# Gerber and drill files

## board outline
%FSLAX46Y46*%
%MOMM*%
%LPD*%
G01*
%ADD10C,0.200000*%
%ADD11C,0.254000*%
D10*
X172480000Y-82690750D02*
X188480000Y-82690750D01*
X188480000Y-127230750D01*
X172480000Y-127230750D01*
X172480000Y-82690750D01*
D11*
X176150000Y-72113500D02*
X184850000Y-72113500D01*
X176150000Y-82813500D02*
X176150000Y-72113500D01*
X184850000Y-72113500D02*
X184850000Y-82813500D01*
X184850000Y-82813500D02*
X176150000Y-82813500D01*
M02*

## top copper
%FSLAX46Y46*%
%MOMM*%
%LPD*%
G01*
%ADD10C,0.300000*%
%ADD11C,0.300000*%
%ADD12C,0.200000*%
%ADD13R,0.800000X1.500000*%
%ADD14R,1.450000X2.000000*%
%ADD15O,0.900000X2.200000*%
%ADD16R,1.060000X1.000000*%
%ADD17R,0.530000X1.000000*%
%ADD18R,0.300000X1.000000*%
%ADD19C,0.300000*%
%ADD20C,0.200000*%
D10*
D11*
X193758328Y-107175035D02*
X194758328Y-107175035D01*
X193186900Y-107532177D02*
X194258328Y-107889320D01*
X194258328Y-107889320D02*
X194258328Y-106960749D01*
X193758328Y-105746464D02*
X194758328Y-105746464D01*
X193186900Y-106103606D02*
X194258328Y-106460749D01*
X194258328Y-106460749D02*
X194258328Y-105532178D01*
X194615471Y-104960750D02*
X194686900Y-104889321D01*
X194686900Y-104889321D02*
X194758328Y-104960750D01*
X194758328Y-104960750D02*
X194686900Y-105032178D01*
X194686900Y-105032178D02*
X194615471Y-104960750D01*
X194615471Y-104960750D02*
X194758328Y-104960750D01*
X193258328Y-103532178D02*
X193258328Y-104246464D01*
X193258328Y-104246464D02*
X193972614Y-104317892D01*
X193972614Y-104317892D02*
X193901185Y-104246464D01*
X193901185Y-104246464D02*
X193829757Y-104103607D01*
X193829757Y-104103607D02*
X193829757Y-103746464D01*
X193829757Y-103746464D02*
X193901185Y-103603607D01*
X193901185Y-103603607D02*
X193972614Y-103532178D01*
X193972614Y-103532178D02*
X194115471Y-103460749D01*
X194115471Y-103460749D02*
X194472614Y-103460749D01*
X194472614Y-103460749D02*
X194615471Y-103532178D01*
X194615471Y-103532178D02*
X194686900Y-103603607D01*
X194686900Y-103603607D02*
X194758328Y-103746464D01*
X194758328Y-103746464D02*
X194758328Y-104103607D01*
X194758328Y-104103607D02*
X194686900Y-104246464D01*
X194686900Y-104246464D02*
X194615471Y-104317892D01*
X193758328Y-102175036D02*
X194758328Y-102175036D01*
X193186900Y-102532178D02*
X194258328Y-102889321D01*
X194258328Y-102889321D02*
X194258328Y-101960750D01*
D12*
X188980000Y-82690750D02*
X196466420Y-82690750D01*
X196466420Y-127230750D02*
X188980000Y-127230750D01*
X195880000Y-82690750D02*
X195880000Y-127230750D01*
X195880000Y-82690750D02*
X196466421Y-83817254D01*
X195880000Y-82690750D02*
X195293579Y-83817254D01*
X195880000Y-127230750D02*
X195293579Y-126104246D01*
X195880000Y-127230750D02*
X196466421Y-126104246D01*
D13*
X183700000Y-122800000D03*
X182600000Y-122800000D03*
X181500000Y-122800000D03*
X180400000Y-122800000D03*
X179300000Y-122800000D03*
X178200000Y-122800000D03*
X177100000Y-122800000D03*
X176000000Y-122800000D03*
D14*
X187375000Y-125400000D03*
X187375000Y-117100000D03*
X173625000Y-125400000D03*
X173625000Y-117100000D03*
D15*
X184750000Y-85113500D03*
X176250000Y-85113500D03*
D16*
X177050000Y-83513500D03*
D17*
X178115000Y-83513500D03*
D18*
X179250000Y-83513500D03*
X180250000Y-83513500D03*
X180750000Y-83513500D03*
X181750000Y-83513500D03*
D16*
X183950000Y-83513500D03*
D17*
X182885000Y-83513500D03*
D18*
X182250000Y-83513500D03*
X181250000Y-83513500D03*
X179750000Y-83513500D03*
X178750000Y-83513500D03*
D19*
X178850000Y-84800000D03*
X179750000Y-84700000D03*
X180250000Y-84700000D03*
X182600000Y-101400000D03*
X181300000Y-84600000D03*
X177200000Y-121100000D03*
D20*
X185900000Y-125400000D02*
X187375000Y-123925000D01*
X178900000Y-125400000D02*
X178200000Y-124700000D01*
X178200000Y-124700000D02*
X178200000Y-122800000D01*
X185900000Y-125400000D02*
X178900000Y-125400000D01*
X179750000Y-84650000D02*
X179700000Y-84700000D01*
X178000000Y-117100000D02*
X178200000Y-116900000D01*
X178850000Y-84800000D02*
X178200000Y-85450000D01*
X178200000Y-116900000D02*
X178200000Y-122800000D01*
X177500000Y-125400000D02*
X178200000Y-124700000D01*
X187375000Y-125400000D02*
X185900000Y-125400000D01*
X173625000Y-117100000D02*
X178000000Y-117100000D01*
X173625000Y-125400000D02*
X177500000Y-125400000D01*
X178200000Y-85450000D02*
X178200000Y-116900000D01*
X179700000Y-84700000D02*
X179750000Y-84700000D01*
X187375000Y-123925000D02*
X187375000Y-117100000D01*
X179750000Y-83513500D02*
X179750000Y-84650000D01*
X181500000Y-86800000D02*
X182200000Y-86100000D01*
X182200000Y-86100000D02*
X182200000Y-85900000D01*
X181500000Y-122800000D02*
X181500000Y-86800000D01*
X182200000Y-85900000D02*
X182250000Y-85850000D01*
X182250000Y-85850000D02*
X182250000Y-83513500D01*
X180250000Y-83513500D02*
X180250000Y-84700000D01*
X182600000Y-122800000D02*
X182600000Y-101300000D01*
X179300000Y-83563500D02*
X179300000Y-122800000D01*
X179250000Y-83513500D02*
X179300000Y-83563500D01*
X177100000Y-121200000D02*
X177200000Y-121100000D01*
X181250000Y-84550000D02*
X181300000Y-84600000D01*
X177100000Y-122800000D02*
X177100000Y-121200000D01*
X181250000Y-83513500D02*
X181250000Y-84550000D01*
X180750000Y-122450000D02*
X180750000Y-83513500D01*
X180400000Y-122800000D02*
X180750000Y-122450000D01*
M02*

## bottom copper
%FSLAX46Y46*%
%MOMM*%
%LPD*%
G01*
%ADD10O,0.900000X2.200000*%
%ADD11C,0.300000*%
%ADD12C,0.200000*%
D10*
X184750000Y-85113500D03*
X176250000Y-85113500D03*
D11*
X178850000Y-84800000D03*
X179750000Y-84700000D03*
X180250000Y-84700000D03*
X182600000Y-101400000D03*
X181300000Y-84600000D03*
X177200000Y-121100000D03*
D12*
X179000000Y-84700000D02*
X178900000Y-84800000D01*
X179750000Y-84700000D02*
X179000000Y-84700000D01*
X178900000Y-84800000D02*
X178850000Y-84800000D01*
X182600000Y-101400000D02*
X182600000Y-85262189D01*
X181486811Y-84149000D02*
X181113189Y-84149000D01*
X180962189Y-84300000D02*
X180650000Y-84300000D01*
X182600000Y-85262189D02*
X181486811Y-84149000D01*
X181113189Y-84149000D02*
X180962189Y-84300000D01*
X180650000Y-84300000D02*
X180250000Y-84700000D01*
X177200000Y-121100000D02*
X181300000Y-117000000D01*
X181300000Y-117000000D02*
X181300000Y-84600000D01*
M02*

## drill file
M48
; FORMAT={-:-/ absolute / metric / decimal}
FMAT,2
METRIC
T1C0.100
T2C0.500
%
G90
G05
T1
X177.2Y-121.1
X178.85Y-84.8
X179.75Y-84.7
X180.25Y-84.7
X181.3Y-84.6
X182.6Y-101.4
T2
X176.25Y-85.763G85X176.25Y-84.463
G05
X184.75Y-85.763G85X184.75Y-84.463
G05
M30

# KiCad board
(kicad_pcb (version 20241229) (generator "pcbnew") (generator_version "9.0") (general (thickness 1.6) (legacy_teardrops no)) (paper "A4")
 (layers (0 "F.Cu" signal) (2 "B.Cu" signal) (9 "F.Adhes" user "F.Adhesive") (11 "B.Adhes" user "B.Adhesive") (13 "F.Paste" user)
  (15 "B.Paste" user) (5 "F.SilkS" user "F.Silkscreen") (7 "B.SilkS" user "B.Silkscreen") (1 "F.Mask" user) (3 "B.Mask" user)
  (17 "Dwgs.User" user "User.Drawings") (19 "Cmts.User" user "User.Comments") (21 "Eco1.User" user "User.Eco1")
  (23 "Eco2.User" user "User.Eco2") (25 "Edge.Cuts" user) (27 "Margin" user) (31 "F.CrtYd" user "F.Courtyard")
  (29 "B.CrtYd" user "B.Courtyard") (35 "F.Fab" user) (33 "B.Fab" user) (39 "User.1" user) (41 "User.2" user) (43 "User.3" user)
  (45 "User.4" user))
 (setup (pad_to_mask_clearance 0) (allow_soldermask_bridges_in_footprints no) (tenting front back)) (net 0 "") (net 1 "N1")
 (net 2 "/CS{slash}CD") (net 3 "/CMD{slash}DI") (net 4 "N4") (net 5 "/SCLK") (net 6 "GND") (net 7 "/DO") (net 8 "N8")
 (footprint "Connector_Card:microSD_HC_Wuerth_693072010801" (layer "F.Cu") (at 180.5 121.25 180)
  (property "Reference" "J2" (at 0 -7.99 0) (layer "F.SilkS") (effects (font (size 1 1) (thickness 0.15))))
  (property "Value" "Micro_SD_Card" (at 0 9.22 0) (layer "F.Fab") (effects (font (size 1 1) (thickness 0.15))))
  (pad "1" smd rect (at -3.2 -1.55 180) (size 0.8 1.5) (layers "F.Cu" "F.Mask" "F.Paste") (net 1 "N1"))
  (pad "2" smd rect (at -2.1 -1.55 180) (size 0.8 1.5) (layers "F.Cu" "F.Mask" "F.Paste") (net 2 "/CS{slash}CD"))
  (pad "3" smd rect (at -1 -1.55 180) (size 0.8 1.5) (layers "F.Cu" "F.Mask" "F.Paste") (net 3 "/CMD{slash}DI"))
  (pad "4" smd rect (at 0.1 -1.55 180) (size 0.8 1.5) (layers "F.Cu" "F.Mask" "F.Paste") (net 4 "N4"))
  (pad "5" smd rect (at 1.2 -1.55 180) (size 0.8 1.5) (layers "F.Cu" "F.Mask" "F.Paste") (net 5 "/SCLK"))
  (pad "6" smd rect (at 2.3 -1.55 180) (size 0.8 1.5) (layers "F.Cu" "F.Mask" "F.Paste") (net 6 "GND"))
  (pad "7" smd rect (at 3.4 -1.55 180) (size 0.8 1.5) (layers "F.Cu" "F.Mask" "F.Paste") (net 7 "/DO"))
  (pad "8" smd rect (at 4.5 -1.55 180) (size 0.8 1.5) (layers "F.Cu" "F.Mask" "F.Paste") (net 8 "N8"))
  (pad "9" smd rect (at -6.875 -4.15 180) (size 1.45 2) (layers "F.Cu" "F.Mask" "F.Paste") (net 6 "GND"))
  (pad "9" smd rect (at -6.875 4.15 180) (size 1.45 2) (layers "F.Cu" "F.Mask" "F.Paste") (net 6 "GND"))
  (pad "9" smd rect (at 6.875 -4.15 180) (size 1.45 2) (layers "F.Cu" "F.Mask" "F.Paste") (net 6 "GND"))
  (pad "9" smd rect (at 6.875 4.15 180) (size 1.45 2) (layers "F.Cu" "F.Mask" "F.Paste") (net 6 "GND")))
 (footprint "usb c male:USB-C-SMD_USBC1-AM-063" (layer "F.Cu") (at 180.5 84.3135 180)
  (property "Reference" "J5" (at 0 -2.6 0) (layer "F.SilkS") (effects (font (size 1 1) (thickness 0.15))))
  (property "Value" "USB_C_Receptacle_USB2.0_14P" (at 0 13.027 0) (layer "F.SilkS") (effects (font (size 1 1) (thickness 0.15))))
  (fp_line (start 4.35 12.2) (end -4.35 12.2) (stroke (width 0.254) (type default)) (layer "Edge.Cuts"))
  (fp_line (start 4.35 1.5) (end 4.35 12.2) (stroke (width 0.254) (type default)) (layer "Edge.Cuts"))
  (fp_line (start -4.35 12.2) (end -4.35 1.5) (stroke (width 0.254) (type default)) (layer "Edge.Cuts"))
  (fp_line (start -4.35 1.5) (end 4.35 1.5) (stroke (width 0.254) (type default)) (layer "Edge.Cuts"))
  (pad "1" thru_hole oval (at -4.25 -0.8 180) (size 0.9 2.2) (drill oval 0.5 1.8) (layers "*.Cu" "*.Mask") (remove_unused_layers no))
  (pad "2" thru_hole oval (at 4.25 -0.8 180) (size 0.9 2.2) (drill oval 0.5 1.8) (layers "*.Cu" "*.Mask") (remove_unused_layers no))
  (pad "A1B12" smd rect (at 3.45 0.8) (size 1.06 1) (layers "F.Cu" "F.Mask" "F.Paste"))
  (pad "A4B9" smd rect (at 2.385 0.8) (size 0.53 1) (layers "F.Cu" "F.Mask" "F.Paste"))
  (pad "A5" smd rect (at 1.25 0.8) (size 0.3 1) (layers "F.Cu" "F.Mask" "F.Paste") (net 5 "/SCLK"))
  (pad "A6" smd rect (at 0.25 0.8 180) (size 0.3 1) (layers "F.Cu" "F.Mask" "F.Paste") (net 2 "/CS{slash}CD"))
  (pad "A7" smd rect (at -0.25 0.8) (size 0.3 1) (layers "F.Cu" "F.Mask" "F.Paste") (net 4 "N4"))
  (pad "A8" smd rect (at -1.25 0.8) (size 0.3 1) (layers "F.Cu" "F.Mask" "F.Paste"))
  (pad "B1A12" smd rect (at -3.45 0.8) (size 1.06 1) (layers "F.Cu" "F.Mask" "F.Paste"))
  (pad "B4A9" smd rect (at -2.385 0.8) (size 0.53 1) (layers "F.Cu" "F.Mask" "F.Paste"))
  (pad "B5" smd rect (at -1.75 0.8) (size 0.3 1) (layers "F.Cu" "F.Mask" "F.Paste") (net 3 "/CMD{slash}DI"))
  (pad "B6" smd rect (at -0.75 0.8 180) (size 0.3 1) (layers "F.Cu" "F.Mask" "F.Paste") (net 7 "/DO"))
  (pad "B7" smd rect (at 0.75 0.8) (size 0.3 1) (layers "F.Cu" "F.Mask" "F.Paste") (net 6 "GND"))
  (pad "B8" smd rect (at 1.75 0.8) (size 0.3 1) (layers "F.Cu" "F.Mask" "F.Paste")))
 (gr_rect (start 172.48 82.69075) (end 188.48 127.23075) (stroke (width 0.2) (type solid)) (fill no) (layer "Edge.Cuts"))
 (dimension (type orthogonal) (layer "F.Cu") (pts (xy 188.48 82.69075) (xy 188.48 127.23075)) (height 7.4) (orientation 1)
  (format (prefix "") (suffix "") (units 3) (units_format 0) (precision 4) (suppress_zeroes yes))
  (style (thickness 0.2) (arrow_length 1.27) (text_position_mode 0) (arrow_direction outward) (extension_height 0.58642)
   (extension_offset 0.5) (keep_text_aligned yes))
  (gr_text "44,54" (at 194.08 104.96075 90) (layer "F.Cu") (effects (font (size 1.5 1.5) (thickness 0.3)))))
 (segment (start 185.9 125.4) (end 187.375 123.925) (width 0.2) (layer "F.Cu") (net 6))
 (segment (start 178.9 125.4) (end 178.2 124.7) (width 0.2) (layer "F.Cu") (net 6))
 (segment (start 178.2 124.7) (end 178.2 122.8) (width 0.2) (layer "F.Cu") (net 6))
 (segment (start 185.9 125.4) (end 178.9 125.4) (width 0.2) (layer "F.Cu") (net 6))
 (segment (start 179.75 84.65) (end 179.7 84.7) (width 0.2) (layer "F.Cu") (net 6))
 (segment (start 178 117.1) (end 178.2 116.9) (width 0.2) (layer "F.Cu") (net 6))
 (segment (start 178.85 84.8) (end 178.2 85.45) (width 0.2) (layer "F.Cu") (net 6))
 (segment (start 178.2 116.9) (end 178.2 122.8) (width 0.2) (layer "F.Cu") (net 6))
 (segment (start 177.5 125.4) (end 178.2 124.7) (width 0.2) (layer "F.Cu") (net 6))
 (segment (start 187.375 125.4) (end 185.9 125.4) (width 0.2) (layer "F.Cu") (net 6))
 (segment (start 173.625 117.1) (end 178 117.1) (width 0.2) (layer "F.Cu") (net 6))
 (segment (start 173.625 125.4) (end 177.5 125.4) (width 0.2) (layer "F.Cu") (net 6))
 (segment (start 178.2 85.45) (end 178.2 116.9) (width 0.2) (layer "F.Cu") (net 6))
 (segment (start 179.7 84.7) (end 179.75 84.7) (width 0.2) (layer "F.Cu") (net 6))
 (segment (start 187.375 123.925) (end 187.375 117.1) (width 0.2) (layer "F.Cu") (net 6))
 (segment (start 179.75 83.5135) (end 179.75 84.65) (width 0.2) (layer "F.Cu") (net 6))
 (via micro (at 178.85 84.8) (size 0.3) (drill 0.1) (layers "F.Cu" "B.Cu") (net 6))
 (via micro (at 179.75 84.7) (size 0.3) (drill 0.1) (layers "F.Cu" "B.Cu") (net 6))
 (segment (start 179 84.7) (end 178.9 84.8) (width 0.2) (layer "B.Cu") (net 6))
 (segment (start 179.75 84.7) (end 179 84.7) (width 0.2) (layer "B.Cu") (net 6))
 (segment (start 178.9 84.8) (end 178.85 84.8) (width 0.2) (layer "B.Cu") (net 6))
 (segment (start 181.5 86.8) (end 182.2 86.1) (width 0.2) (layer "F.Cu") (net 3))
 (segment (start 182.2 86.1) (end 182.2 85.9) (width 0.2) (layer "F.Cu") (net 3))
 (segment (start 181.5 122.8) (end 181.5 86.8) (width 0.2) (layer "F.Cu") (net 3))
 (segment (start 182.2 85.9) (end 182.25 85.85) (width 0.2) (layer "F.Cu") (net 3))
 (segment (start 182.25 85.85) (end 182.25 83.5135) (width 0.2) (layer "F.Cu") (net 3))
 (segment (start 180.25 83.5135) (end 180.25 84.7) (width 0.2) (layer "F.Cu") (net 2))
 (segment (start 182.6 122.8) (end 182.6 101.3) (width 0.2) (layer "F.Cu") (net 2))
 (via micro (at 180.25 84.7) (size 0.3) (drill 0.1) (layers "F.Cu" "B.Cu") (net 2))
 (via micro (at 182.6 101.4) (size 0.3) (drill 0.1) (layers "F.Cu" "B.Cu") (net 2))
 (segment (start 182.6 101.4) (end 182.6 85.262189) (width 0.2) (layer "B.Cu") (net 2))
 (segment (start 181.486811 84.149) (end 181.113189 84.149) (width 0.2) (layer "B.Cu") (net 2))
 (segment (start 180.962189 84.3) (end 180.65 84.3) (width 0.2) (layer "B.Cu") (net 2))
 (segment (start 182.6 85.262189) (end 181.486811 84.149) (width 0.2) (layer "B.Cu") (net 2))
 (segment (start 181.113189 84.149) (end 180.962189 84.3) (width 0.2) (layer "B.Cu") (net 2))
 (segment (start 180.65 84.3) (end 180.25 84.7) (width 0.2) (layer "B.Cu") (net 2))
 (segment (start 179.3 83.5635) (end 179.3 122.8) (width 0.2) (layer "F.Cu") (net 5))
 (segment (start 179.25 83.5135) (end 179.3 83.5635) (width 0.2) (layer "F.Cu") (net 5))
 (segment (start 177.1 121.2) (end 177.2 121.1) (width 0.2) (layer "F.Cu") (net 7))
 (segment (start 181.25 84.55) (end 181.3 84.6) (width 0.2) (layer "F.Cu") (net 7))
 (segment (start 177.1 122.8) (end 177.1 121.2) (width 0.2) (layer "F.Cu") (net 7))
 (segment (start 181.25 83.5135) (end 181.25 84.55) (width 0.2) (layer "F.Cu") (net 7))
 (via micro (at 181.3 84.6) (size 0.3) (drill 0.1) (layers "F.Cu" "B.Cu") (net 7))
 (via micro (at 177.2 121.1) (size 0.3) (drill 0.1) (layers "F.Cu" "B.Cu") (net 7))
 (segment (start 177.2 121.1) (end 181.3 117) (width 0.2) (layer "B.Cu") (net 7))
 (segment (start 181.3 117) (end 181.3 84.6) (width 0.2) (layer "B.Cu") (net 7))
 (segment (start 180.75 122.45) (end 180.75 83.5135) (width 0.2) (layer "F.Cu") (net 4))
 (segment (start 180.4 122.8) (end 180.75 122.45) (width 0.2) (layer "F.Cu") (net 4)))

